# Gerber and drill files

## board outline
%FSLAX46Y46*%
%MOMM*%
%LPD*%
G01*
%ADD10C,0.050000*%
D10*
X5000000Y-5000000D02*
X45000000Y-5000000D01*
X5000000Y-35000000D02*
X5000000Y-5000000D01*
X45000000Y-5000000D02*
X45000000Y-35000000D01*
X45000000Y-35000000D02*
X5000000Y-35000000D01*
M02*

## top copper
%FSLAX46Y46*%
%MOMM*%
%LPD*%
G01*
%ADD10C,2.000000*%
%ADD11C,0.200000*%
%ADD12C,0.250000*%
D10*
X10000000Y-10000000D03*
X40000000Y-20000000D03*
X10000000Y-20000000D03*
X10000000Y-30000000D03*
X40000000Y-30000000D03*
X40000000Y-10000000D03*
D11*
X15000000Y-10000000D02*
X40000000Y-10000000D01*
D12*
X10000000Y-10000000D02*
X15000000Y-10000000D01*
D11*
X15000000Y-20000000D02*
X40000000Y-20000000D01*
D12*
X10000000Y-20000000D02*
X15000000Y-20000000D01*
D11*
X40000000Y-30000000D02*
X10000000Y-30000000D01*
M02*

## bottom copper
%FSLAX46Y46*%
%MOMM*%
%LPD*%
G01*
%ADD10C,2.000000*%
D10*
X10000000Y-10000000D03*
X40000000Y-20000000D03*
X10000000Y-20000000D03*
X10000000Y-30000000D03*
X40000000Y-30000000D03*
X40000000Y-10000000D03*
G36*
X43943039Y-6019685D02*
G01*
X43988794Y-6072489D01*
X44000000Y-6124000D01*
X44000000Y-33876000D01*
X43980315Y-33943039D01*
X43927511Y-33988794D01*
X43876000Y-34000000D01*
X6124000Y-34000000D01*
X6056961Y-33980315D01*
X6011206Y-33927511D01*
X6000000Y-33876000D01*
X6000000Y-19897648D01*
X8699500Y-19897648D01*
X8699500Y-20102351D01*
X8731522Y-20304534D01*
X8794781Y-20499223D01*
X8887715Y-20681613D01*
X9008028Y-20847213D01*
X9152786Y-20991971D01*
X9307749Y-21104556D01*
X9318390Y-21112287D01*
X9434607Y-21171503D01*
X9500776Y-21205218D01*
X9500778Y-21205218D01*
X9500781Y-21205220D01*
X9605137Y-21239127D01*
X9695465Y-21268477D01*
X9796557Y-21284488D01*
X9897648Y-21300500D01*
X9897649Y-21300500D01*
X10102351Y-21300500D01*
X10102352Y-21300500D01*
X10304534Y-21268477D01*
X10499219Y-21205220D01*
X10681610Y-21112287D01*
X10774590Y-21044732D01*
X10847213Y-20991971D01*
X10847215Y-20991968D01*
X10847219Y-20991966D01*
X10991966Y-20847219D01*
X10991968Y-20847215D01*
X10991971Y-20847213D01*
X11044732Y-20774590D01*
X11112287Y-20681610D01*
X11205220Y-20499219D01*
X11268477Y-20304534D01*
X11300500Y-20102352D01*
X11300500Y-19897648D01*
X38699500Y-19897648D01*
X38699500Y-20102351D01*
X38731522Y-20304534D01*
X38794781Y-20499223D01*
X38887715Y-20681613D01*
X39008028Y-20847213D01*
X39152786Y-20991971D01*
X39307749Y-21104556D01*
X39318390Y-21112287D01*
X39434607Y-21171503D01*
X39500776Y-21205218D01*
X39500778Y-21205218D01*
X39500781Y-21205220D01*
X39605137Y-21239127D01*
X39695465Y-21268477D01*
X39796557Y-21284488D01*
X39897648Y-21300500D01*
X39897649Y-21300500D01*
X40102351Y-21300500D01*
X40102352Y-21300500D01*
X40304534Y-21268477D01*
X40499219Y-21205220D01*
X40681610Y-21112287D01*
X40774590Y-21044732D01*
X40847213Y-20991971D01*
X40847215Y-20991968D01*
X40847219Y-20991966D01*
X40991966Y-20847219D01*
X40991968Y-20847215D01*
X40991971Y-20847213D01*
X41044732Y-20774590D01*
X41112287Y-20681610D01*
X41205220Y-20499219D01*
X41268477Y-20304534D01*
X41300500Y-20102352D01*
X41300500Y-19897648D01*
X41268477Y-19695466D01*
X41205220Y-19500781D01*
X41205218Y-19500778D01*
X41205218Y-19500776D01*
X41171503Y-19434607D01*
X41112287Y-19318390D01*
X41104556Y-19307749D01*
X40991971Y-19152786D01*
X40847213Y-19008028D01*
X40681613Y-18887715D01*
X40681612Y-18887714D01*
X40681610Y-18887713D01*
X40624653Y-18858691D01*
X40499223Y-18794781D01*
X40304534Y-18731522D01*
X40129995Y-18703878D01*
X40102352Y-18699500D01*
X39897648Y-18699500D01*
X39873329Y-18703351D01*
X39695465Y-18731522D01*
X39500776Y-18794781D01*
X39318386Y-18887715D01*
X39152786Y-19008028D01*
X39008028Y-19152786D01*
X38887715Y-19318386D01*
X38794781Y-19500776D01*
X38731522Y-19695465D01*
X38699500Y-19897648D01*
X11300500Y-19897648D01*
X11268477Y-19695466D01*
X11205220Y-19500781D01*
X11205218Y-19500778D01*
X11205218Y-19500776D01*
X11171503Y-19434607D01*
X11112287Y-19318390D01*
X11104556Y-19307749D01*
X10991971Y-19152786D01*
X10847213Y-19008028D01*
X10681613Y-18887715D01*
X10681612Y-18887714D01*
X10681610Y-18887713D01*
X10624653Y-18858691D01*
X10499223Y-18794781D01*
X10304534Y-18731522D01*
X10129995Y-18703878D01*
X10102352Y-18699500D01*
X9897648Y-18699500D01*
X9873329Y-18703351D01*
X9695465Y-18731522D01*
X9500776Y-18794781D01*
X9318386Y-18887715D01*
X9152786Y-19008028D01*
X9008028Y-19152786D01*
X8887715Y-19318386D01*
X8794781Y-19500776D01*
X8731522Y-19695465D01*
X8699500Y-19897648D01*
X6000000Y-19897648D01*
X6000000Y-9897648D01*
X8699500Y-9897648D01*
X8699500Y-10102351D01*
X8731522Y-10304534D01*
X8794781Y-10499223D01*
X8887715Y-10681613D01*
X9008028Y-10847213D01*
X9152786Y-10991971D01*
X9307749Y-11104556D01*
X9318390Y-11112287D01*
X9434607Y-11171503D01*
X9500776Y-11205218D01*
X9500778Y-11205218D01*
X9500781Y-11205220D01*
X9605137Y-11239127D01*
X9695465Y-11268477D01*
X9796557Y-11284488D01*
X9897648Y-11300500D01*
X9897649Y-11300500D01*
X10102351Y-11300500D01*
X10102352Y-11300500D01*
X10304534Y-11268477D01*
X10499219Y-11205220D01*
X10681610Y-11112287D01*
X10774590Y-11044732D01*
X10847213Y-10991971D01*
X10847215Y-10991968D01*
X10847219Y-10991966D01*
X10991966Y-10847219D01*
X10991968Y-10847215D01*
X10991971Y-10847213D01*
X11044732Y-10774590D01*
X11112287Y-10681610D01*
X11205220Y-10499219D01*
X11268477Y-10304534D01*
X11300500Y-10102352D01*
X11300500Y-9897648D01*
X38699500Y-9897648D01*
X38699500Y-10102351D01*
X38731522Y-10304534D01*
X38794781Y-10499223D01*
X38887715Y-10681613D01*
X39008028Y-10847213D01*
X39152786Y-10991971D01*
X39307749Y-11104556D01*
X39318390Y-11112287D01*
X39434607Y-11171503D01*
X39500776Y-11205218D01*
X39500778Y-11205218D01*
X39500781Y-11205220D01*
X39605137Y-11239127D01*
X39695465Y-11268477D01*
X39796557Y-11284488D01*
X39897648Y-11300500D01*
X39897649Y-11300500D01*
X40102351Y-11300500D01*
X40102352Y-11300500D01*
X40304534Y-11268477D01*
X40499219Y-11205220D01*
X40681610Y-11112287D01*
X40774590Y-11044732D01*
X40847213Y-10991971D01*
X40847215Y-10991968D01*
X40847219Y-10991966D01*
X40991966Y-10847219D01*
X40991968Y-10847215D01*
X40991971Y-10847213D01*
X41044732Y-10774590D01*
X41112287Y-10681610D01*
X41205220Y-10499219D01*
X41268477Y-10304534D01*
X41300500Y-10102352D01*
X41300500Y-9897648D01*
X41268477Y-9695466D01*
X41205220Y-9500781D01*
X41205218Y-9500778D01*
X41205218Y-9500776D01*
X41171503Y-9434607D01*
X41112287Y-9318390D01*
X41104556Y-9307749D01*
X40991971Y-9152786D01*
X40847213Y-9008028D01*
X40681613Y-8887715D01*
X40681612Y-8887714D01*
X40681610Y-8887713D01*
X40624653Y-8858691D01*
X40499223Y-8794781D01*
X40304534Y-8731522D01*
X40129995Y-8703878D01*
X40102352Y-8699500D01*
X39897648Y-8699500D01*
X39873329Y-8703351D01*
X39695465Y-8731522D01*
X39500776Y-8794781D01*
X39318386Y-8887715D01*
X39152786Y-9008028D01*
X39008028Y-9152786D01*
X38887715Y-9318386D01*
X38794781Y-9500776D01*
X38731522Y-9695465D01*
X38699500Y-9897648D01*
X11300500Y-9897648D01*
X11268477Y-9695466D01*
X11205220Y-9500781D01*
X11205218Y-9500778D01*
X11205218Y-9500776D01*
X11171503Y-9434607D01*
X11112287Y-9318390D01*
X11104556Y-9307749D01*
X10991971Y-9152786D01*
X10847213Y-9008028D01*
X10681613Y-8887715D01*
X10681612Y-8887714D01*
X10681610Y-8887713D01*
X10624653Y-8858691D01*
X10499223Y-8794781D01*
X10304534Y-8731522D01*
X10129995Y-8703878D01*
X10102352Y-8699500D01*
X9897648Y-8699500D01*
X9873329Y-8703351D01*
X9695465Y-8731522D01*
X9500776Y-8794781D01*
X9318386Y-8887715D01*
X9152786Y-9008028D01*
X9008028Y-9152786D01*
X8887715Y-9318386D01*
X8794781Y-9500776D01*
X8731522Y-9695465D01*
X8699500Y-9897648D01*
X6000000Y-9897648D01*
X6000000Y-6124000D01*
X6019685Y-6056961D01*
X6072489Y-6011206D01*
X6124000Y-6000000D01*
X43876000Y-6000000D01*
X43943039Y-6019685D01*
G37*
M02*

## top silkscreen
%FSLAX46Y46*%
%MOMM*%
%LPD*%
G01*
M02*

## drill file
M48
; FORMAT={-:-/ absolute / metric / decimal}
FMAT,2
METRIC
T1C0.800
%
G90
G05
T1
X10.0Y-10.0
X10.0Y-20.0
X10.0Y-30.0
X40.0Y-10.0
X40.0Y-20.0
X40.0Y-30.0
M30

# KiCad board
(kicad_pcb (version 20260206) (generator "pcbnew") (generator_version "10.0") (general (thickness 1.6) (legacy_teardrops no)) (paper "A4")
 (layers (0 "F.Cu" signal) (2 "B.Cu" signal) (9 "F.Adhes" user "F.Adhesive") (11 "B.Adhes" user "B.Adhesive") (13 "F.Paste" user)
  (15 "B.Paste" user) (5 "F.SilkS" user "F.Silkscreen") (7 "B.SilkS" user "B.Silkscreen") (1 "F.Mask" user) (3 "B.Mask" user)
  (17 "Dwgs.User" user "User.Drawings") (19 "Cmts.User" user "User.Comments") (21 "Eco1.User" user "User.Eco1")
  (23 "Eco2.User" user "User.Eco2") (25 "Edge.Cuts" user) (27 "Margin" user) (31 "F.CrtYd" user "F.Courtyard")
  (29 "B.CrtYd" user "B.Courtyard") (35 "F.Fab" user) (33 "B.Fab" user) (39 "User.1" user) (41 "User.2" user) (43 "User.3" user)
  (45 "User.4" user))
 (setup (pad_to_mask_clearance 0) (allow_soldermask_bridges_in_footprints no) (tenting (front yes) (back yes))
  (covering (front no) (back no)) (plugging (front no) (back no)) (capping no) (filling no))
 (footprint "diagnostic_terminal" (layer "F.Cu") (at 10 10)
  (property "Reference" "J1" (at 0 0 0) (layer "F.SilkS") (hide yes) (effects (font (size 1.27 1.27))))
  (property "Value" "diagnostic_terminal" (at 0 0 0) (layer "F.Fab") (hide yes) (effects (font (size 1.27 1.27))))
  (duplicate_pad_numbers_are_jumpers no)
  (pad "1" thru_hole circle (at 0 0) (size 2 2) (drill 0.8) (layers "*.Cu") (remove_unused_layers no) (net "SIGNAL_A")))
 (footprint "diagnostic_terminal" (layer "F.Cu") (at 40 20)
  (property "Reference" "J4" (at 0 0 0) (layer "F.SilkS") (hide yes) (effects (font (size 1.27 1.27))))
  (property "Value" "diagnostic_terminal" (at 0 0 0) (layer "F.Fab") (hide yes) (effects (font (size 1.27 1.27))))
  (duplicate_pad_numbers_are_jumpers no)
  (pad "1" thru_hole circle (at 0 0) (size 2 2) (drill 0.8) (layers "*.Cu") (remove_unused_layers no) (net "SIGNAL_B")))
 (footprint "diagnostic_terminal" (layer "F.Cu") (at 10 20)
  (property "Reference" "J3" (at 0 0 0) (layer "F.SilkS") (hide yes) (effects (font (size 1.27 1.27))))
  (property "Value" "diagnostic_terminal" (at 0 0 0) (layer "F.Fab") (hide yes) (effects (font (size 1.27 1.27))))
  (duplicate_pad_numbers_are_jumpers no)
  (pad "1" thru_hole circle (at 0 0) (size 2 2) (drill 0.8) (layers "*.Cu") (remove_unused_layers no) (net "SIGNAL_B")))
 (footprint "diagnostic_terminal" (layer "F.Cu") (at 10 30)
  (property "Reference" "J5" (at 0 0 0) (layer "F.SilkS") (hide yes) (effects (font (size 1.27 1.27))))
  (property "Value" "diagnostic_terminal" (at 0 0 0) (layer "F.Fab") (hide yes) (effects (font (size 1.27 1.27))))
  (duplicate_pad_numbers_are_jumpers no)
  (pad "1" thru_hole circle (at 0 0) (size 2 2) (drill 0.8) (layers "*.Cu") (remove_unused_layers no) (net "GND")))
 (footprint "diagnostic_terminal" (layer "F.Cu") (at 40 30)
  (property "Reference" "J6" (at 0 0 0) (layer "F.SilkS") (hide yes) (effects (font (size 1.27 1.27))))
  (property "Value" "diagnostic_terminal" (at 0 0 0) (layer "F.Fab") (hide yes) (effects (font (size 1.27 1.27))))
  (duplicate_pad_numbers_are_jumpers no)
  (pad "1" thru_hole circle (at 0 0) (size 2 2) (drill 0.8) (layers "*.Cu") (remove_unused_layers no) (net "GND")))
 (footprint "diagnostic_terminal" (layer "F.Cu") (at 40 10)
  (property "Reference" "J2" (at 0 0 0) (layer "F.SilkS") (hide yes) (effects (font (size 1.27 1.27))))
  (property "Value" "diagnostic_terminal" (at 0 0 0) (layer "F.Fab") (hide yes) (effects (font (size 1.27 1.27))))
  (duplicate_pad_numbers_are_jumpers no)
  (pad "1" thru_hole circle (at 0 0) (size 2 2) (drill 0.8) (layers "*.Cu") (remove_unused_layers no) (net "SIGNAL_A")))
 (gr_line (start 5 5) (end 45 5) (stroke (width 0.05) (type default)) (layer "Edge.Cuts"))
 (gr_line (start 5 35) (end 5 5) (stroke (width 0.05) (type default)) (layer "Edge.Cuts"))
 (gr_line (start 45 5) (end 45 35) (stroke (width 0.05) (type default)) (layer "Edge.Cuts"))
 (gr_line (start 45 35) (end 5 35) (stroke (width 0.05) (type default)) (layer "Edge.Cuts"))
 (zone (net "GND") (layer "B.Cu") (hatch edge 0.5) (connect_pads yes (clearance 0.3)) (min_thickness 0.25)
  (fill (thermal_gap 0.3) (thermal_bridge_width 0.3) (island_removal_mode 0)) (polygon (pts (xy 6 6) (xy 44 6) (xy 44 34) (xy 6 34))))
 (segment (start 15 10) (end 40 10) (width 0.2) (layer "F.Cu") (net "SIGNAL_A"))
 (segment (start 10 10) (end 15 10) (width 0.25) (layer "F.Cu") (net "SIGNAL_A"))
 (segment (start 15 20) (end 40 20) (width 0.2) (layer "F.Cu") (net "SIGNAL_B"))
 (segment (start 10 20) (end 15 20) (width 0.25) (layer "F.Cu") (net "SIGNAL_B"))
 (segment (start 40 30) (end 10 30) (width 0.2) (layer "F.Cu") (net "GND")))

